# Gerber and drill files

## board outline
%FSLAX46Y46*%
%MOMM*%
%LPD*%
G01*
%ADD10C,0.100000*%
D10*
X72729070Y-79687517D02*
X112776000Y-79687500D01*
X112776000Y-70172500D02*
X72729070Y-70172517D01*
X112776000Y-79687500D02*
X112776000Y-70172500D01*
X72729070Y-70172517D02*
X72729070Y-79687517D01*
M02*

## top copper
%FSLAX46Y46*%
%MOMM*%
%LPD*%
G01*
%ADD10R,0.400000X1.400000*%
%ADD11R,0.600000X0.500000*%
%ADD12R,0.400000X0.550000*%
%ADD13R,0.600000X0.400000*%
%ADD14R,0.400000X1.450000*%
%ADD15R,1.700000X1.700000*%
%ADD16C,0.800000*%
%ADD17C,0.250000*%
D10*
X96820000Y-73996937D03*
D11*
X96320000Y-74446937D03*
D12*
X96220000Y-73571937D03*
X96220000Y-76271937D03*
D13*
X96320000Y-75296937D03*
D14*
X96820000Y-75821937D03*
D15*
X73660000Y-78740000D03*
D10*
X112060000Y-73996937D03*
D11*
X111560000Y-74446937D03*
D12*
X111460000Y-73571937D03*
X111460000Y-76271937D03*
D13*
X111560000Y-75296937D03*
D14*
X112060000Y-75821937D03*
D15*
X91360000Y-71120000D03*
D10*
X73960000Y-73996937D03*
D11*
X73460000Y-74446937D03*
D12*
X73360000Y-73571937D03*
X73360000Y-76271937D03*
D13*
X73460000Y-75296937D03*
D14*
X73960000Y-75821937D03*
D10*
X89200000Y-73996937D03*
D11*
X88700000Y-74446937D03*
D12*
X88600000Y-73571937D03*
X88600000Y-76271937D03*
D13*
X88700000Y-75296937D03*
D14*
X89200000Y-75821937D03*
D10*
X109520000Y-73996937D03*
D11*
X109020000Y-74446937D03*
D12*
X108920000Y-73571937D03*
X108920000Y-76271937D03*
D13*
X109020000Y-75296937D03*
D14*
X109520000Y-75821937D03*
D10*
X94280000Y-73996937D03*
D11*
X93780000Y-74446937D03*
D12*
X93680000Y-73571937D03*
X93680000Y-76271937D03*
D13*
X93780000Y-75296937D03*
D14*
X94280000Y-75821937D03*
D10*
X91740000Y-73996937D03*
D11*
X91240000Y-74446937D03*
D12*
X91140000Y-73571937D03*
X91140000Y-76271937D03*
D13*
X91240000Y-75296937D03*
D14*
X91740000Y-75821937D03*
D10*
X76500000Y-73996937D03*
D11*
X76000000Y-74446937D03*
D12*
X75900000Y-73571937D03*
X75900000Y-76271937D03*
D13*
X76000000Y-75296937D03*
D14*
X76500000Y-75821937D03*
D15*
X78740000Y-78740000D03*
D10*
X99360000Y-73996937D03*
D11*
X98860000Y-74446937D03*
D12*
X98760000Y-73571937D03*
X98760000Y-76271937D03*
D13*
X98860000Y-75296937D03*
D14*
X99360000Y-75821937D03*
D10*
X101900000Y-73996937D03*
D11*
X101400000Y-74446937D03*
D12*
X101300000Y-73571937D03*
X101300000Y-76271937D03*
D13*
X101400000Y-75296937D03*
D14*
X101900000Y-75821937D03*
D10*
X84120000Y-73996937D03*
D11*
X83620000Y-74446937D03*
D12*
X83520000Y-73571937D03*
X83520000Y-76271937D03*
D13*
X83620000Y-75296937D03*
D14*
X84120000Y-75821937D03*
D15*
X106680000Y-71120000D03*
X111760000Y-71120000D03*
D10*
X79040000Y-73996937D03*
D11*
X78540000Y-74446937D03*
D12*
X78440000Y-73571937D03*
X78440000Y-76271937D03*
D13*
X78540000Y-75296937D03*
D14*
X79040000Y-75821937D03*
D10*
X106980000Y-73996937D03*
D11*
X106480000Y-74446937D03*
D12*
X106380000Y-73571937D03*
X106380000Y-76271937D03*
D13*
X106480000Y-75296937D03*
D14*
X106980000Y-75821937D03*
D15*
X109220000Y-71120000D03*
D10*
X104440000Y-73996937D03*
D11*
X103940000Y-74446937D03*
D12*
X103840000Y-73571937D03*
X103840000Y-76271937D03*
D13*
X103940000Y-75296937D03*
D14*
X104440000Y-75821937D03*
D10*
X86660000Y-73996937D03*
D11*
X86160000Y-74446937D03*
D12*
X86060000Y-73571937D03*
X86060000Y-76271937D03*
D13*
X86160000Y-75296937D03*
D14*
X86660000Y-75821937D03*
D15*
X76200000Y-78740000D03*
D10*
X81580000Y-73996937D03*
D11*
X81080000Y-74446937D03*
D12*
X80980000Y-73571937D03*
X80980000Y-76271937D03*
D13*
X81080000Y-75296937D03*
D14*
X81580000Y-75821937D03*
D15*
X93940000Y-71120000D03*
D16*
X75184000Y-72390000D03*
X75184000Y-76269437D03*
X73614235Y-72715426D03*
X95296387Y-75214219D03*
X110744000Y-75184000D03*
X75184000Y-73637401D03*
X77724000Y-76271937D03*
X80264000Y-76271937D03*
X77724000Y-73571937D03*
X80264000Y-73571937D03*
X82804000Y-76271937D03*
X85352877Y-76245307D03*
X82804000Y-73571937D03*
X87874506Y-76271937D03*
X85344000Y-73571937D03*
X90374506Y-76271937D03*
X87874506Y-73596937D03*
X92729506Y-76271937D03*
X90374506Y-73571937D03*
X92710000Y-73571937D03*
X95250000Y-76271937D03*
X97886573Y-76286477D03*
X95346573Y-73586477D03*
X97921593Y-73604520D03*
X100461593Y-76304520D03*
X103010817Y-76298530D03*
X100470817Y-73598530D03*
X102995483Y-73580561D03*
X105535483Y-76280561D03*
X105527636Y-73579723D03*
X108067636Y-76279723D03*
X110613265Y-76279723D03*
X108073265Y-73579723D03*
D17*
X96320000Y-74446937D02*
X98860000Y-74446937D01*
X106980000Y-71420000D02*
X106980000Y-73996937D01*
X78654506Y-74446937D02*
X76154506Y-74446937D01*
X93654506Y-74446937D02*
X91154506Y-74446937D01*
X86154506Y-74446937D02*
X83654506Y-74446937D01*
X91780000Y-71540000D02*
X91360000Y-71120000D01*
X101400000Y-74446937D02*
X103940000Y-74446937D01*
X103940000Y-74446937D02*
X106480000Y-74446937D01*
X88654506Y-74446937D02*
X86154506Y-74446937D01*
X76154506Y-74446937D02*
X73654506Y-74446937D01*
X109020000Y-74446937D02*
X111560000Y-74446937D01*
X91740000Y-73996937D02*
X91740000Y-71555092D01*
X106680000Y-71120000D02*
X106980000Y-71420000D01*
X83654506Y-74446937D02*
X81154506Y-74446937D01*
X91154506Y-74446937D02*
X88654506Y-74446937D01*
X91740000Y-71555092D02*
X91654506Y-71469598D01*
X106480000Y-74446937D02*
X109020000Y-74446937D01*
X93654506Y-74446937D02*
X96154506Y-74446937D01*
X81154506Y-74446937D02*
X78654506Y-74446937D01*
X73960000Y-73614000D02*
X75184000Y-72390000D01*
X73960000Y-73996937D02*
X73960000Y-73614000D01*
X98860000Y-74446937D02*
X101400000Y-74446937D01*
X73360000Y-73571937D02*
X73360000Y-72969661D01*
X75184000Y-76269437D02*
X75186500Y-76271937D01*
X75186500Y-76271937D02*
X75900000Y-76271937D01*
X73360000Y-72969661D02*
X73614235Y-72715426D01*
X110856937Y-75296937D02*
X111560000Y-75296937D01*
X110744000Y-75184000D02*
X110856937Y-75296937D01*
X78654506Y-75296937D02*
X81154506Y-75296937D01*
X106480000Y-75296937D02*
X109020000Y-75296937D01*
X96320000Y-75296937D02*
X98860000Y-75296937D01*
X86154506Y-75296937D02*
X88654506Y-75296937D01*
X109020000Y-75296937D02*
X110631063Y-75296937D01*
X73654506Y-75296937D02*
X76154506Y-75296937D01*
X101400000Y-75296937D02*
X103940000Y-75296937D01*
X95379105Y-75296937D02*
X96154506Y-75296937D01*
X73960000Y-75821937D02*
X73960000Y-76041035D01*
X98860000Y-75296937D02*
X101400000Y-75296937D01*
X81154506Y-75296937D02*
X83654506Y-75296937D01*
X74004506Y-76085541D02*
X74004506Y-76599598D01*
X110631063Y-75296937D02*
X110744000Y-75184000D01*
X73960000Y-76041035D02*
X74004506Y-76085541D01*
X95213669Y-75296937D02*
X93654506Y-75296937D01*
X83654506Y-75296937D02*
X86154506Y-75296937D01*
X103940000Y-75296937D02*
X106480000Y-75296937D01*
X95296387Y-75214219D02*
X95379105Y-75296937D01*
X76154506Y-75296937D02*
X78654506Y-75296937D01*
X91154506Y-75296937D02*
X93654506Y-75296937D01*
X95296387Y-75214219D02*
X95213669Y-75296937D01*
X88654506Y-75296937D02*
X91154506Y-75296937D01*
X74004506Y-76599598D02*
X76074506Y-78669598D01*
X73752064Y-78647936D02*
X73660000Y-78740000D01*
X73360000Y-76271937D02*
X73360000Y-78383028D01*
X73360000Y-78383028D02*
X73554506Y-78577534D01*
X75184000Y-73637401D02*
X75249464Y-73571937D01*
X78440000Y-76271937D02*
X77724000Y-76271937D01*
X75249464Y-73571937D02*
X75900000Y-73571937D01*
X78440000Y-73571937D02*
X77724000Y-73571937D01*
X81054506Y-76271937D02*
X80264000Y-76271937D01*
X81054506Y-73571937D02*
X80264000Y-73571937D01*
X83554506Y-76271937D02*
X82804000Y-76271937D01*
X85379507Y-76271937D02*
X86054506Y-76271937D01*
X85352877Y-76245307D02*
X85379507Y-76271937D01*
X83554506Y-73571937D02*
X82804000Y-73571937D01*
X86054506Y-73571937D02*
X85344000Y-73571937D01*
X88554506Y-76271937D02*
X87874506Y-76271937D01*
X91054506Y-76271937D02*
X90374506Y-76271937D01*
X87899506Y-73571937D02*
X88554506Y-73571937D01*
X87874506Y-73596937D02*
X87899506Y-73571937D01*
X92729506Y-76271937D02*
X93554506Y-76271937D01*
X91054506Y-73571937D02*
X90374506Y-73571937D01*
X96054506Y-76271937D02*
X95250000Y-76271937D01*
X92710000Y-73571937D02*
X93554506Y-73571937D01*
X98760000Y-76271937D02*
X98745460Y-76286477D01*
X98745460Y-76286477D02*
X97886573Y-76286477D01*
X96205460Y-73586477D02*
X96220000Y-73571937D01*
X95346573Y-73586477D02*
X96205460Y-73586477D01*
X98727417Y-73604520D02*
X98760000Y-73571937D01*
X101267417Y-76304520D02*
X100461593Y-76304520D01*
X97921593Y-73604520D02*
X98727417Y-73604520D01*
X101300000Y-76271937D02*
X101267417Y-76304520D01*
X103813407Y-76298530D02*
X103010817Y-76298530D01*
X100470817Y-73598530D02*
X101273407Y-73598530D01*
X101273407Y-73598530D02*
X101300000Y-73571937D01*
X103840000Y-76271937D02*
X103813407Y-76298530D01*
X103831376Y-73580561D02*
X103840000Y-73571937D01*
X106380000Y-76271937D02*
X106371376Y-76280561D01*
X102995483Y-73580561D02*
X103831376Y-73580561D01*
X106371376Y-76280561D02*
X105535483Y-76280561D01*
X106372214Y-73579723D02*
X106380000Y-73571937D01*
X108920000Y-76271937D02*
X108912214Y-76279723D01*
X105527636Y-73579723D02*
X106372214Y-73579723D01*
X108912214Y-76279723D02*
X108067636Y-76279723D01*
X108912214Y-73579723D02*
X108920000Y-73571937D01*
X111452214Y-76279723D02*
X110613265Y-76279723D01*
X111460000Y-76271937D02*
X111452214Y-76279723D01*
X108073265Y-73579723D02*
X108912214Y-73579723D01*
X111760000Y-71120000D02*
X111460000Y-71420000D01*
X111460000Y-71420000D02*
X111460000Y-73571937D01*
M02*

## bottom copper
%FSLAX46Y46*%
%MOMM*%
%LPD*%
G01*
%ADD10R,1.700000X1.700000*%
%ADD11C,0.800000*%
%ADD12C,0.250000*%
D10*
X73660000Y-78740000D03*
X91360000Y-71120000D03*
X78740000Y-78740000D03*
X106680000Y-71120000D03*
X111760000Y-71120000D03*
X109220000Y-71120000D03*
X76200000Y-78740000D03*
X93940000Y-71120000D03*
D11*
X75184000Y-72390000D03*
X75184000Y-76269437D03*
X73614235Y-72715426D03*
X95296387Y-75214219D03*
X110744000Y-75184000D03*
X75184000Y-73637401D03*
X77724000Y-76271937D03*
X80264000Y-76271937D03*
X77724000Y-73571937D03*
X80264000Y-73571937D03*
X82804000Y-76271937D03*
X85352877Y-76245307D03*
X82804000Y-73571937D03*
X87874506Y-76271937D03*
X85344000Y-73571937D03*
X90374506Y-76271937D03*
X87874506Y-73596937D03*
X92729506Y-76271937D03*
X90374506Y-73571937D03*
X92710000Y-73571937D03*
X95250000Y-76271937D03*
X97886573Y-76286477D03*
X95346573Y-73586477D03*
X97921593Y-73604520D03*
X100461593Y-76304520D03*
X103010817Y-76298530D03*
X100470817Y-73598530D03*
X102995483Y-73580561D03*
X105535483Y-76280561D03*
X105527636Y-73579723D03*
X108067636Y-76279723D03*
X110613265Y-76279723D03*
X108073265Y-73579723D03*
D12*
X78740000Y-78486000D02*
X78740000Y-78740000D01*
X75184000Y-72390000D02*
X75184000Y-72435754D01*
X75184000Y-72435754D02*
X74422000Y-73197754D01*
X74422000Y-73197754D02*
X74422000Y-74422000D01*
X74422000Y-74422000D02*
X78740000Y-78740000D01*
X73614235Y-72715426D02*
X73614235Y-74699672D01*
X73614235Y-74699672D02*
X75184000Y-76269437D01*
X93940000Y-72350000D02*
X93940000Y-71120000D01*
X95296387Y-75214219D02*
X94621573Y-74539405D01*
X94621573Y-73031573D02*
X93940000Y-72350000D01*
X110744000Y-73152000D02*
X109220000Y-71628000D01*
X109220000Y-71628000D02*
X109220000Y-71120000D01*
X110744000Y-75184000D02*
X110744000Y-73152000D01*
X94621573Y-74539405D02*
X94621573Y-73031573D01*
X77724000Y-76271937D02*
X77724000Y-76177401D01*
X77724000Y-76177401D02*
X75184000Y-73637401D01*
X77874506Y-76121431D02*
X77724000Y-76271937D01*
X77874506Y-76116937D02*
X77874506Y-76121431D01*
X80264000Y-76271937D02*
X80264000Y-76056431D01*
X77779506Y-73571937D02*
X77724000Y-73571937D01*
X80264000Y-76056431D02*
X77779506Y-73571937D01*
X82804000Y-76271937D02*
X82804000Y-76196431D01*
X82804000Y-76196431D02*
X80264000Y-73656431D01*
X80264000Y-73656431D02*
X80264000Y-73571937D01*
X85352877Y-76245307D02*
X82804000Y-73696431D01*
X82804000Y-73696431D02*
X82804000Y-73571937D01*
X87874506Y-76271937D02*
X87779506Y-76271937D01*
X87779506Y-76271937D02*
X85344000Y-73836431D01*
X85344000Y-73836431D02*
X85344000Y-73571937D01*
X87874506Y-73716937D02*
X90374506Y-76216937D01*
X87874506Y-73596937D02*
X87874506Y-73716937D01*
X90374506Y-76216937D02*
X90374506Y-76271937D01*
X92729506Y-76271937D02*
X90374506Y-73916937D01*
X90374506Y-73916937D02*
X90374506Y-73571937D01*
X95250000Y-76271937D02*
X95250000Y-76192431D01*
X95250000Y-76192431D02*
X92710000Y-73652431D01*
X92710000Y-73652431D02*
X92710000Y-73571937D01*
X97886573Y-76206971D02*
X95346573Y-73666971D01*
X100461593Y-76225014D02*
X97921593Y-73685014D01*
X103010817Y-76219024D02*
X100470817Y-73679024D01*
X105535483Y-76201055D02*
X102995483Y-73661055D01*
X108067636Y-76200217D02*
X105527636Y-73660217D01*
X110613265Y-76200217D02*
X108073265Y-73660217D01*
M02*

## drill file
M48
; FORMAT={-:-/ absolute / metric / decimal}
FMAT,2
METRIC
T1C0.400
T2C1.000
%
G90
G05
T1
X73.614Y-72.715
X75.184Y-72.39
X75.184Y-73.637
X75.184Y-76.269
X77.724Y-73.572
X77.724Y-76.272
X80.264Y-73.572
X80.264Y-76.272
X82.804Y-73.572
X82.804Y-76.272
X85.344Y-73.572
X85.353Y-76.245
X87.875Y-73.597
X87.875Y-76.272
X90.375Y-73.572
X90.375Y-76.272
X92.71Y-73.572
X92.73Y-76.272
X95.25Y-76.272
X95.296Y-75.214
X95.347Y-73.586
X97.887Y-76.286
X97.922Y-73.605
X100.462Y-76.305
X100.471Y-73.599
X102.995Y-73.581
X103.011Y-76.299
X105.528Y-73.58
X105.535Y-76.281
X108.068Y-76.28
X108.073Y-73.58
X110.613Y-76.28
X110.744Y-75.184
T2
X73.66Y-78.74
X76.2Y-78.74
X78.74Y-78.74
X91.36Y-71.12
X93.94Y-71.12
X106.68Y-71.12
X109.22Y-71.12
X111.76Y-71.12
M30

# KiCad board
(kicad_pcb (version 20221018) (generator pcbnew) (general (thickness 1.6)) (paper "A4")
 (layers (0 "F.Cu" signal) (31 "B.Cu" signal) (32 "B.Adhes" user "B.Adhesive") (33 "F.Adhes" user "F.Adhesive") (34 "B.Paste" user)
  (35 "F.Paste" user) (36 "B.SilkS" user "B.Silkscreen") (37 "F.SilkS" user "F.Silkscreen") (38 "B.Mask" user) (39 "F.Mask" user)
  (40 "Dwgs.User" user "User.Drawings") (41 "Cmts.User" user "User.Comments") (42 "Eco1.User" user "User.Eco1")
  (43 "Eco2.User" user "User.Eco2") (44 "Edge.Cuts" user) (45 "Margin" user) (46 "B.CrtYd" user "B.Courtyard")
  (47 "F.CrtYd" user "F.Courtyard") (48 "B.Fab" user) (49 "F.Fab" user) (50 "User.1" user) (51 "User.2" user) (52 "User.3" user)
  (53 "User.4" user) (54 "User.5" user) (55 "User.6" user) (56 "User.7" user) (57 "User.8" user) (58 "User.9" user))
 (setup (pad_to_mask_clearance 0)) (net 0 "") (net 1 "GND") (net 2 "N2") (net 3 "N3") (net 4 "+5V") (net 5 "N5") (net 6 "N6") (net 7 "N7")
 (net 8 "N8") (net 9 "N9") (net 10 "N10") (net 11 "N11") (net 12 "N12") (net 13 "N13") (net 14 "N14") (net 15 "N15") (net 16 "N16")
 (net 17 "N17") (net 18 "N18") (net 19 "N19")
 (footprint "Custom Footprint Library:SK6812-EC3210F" (layer "F.Cu") (at 96.52 74.896937 -90)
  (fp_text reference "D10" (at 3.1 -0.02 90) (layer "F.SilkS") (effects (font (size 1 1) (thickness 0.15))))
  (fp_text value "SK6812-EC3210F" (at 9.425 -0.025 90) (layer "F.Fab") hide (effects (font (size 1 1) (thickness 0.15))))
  (pad "1" smd rect (at -0.9 -0.3 90) (size 1.4 0.4) (layers "F.Cu" "F.Paste" "F.Mask") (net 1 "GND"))
  (pad "1" smd rect (at -0.45 0.2 90) (size 0.5 0.6) (layers "F.Cu" "F.Paste" "F.Mask") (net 1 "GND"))
  (pad "2" smd rect (at -1.325 0.3 90) (size 0.55 0.4) (layers "F.Cu" "F.Paste" "F.Mask") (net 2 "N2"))
  (pad "3" smd rect (at 1.375 0.3 90) (size 0.55 0.4) (layers "F.Cu" "F.Paste" "F.Mask") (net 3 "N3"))
  (pad "4" smd rect (at 0.4 0.2 90) (size 0.4 0.6) (layers "F.Cu" "F.Paste" "F.Mask") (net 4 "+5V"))
  (pad "4" smd rect (at 0.925 -0.3 90) (size 1.45 0.4) (layers "F.Cu" "F.Paste" "F.Mask") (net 4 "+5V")))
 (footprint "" (layer "F.Cu") (at 73.66 78.74)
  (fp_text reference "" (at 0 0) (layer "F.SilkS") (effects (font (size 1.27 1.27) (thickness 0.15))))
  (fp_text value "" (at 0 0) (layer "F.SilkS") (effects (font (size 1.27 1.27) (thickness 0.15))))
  (pad "1" thru_hole rect (at 0 0) (size 1.7 1.7) (drill 1) (layers "*.Cu" "*.Mask") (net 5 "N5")))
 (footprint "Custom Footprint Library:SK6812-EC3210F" (layer "F.Cu") (at 111.76 74.896937 -90)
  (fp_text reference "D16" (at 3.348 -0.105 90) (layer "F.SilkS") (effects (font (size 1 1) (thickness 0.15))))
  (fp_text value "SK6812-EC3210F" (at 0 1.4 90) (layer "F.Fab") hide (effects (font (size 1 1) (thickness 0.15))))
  (pad "1" smd rect (at -0.9 -0.3 90) (size 1.4 0.4) (layers "F.Cu" "F.Paste" "F.Mask") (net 1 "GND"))
  (pad "1" smd rect (at -0.45 0.2 90) (size 0.5 0.6) (layers "F.Cu" "F.Paste" "F.Mask") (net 1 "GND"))
  (pad "2" smd rect (at -1.325 0.3 90) (size 0.55 0.4) (layers "F.Cu" "F.Paste" "F.Mask") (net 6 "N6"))
  (pad "3" smd rect (at 1.375 0.3 90) (size 0.55 0.4) (layers "F.Cu" "F.Paste" "F.Mask") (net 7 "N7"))
  (pad "4" smd rect (at 0.4 0.2 90) (size 0.4 0.6) (layers "F.Cu" "F.Paste" "F.Mask") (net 4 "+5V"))
  (pad "4" smd rect (at 0.925 -0.3 90) (size 1.45 0.4) (layers "F.Cu" "F.Paste" "F.Mask") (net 4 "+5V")))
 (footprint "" (layer "F.Cu") (at 91.44 71.12)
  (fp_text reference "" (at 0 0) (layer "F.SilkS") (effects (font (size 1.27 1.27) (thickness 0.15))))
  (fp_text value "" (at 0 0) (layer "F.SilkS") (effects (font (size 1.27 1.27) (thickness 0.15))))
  (pad "1" thru_hole rect (at -0.08 0) (size 1.7 1.7) (drill 1) (layers "*.Cu" "*.Mask") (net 1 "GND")))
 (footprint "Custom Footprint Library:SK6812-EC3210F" (layer "F.Cu") (at 73.66 74.896937 -90)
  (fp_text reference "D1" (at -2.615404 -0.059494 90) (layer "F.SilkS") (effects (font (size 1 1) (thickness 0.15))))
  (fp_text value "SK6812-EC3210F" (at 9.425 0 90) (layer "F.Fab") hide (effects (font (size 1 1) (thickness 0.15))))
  (pad "1" smd rect (at -0.9 -0.3 90) (size 1.4 0.4) (layers "F.Cu" "F.Paste" "F.Mask") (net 1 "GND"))
  (pad "1" smd rect (at -0.45 0.2 90) (size 0.5 0.6) (layers "F.Cu" "F.Paste" "F.Mask") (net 1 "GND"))
  (pad "2" smd rect (at -1.325 0.3 90) (size 0.55 0.4) (layers "F.Cu" "F.Paste" "F.Mask") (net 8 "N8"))
  (pad "3" smd rect (at 1.375 0.3 90) (size 0.55 0.4) (layers "F.Cu" "F.Paste" "F.Mask") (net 5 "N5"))
  (pad "4" smd rect (at 0.4 0.2 90) (size 0.4 0.6) (layers "F.Cu" "F.Paste" "F.Mask") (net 4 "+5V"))
  (pad "4" smd rect (at 0.925 -0.3 90) (size 1.45 0.4) (layers "F.Cu" "F.Paste" "F.Mask") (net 4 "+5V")))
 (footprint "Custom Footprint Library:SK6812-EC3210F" (layer "F.Cu") (at 88.9 74.896937 -90)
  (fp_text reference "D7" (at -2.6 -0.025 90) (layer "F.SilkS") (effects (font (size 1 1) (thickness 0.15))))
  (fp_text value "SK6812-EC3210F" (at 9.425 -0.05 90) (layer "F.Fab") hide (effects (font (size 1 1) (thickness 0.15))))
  (pad "1" smd rect (at -0.9 -0.3 90) (size 1.4 0.4) (layers "F.Cu" "F.Paste" "F.Mask") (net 1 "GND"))
  (pad "1" smd rect (at -0.45 0.2 90) (size 0.5 0.6) (layers "F.Cu" "F.Paste" "F.Mask") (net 1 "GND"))
  (pad "2" smd rect (at -1.325 0.3 90) (size 0.55 0.4) (layers "F.Cu" "F.Paste" "F.Mask") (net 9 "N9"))
  (pad "3" smd rect (at 1.375 0.3 90) (size 0.55 0.4) (layers "F.Cu" "F.Paste" "F.Mask") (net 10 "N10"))
  (pad "4" smd rect (at 0.4 0.2 90) (size 0.4 0.6) (layers "F.Cu" "F.Paste" "F.Mask") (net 4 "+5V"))
  (pad "4" smd rect (at 0.925 -0.3 90) (size 1.45 0.4) (layers "F.Cu" "F.Paste" "F.Mask") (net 4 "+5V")))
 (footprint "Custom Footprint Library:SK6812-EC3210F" (layer "F.Cu") (at 109.22 74.896937 -90)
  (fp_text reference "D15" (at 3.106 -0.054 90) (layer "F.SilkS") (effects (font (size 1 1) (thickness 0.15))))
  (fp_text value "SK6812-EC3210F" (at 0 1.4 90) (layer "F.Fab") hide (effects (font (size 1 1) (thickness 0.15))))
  (pad "1" smd rect (at -0.9 -0.3 90) (size 1.4 0.4) (layers "F.Cu" "F.Paste" "F.Mask") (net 1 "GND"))
  (pad "1" smd rect (at -0.45 0.2 90) (size 0.5 0.6) (layers "F.Cu" "F.Paste" "F.Mask") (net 1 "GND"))
  (pad "2" smd rect (at -1.325 0.3 90) (size 0.55 0.4) (layers "F.Cu" "F.Paste" "F.Mask") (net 7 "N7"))
  (pad "3" smd rect (at 1.375 0.3 90) (size 0.55 0.4) (layers "F.Cu" "F.Paste" "F.Mask") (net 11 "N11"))
  (pad "4" smd rect (at 0.4 0.2 90) (size 0.4 0.6) (layers "F.Cu" "F.Paste" "F.Mask") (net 4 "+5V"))
  (pad "4" smd rect (at 0.925 -0.3 90) (size 1.45 0.4) (layers "F.Cu" "F.Paste" "F.Mask") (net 4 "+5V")))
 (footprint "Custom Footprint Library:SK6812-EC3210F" (layer "F.Cu") (at 93.98 74.896937 -90)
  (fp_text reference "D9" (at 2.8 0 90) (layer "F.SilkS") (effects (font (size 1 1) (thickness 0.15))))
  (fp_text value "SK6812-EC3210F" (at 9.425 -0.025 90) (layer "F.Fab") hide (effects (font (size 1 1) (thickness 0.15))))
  (pad "1" smd rect (at -0.9 -0.3 90) (size 1.4 0.4) (layers "F.Cu" "F.Paste" "F.Mask") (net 1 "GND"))
  (pad "1" smd rect (at -0.45 0.2 90) (size 0.5 0.6) (layers "F.Cu" "F.Paste" "F.Mask") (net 1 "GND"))
  (pad "2" smd rect (at -1.325 0.3 90) (size 0.55 0.4) (layers "F.Cu" "F.Paste" "F.Mask") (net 3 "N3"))
  (pad "3" smd rect (at 1.375 0.3 90) (size 0.55 0.4) (layers "F.Cu" "F.Paste" "F.Mask") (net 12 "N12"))
  (pad "4" smd rect (at 0.4 0.2 90) (size 0.4 0.6) (layers "F.Cu" "F.Paste" "F.Mask") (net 4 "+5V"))
  (pad "4" smd rect (at 0.925 -0.3 90) (size 1.45 0.4) (layers "F.Cu" "F.Paste" "F.Mask") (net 4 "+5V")))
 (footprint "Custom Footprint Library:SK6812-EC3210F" (layer "F.Cu") (at 91.44 74.896937 -90)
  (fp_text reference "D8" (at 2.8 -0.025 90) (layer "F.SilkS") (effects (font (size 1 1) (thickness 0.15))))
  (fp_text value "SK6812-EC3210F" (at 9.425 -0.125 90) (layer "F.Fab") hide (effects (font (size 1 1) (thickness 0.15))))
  (pad "1" smd rect (at -0.9 -0.3 90) (size 1.4 0.4) (layers "F.Cu" "F.Paste" "F.Mask") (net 1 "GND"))
  (pad "1" smd rect (at -0.45 0.2 90) (size 0.5 0.6) (layers "F.Cu" "F.Paste" "F.Mask") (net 1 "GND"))
  (pad "2" smd rect (at -1.325 0.3 90) (size 0.55 0.4) (layers "F.Cu" "F.Paste" "F.Mask") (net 12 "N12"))
  (pad "3" smd rect (at 1.375 0.3 90) (size 0.55 0.4) (layers "F.Cu" "F.Paste" "F.Mask") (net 9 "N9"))
  (pad "4" smd rect (at 0.4 0.2 90) (size 0.4 0.6) (layers "F.Cu" "F.Paste" "F.Mask") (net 4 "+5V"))
  (pad "4" smd rect (at 0.925 -0.3 90) (size 1.45 0.4) (layers "F.Cu" "F.Paste" "F.Mask") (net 4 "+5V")))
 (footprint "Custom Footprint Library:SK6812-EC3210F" (layer "F.Cu") (at 76.2 74.896937 -90)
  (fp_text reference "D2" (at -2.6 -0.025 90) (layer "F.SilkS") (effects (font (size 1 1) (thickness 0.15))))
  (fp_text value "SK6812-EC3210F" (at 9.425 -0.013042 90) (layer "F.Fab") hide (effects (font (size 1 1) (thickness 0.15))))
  (pad "1" smd rect (at -0.9 -0.3 90) (size 1.4 0.4) (layers "F.Cu" "F.Paste" "F.Mask") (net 1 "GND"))
  (pad "1" smd rect (at -0.45 0.2 90) (size 0.5 0.6) (layers "F.Cu" "F.Paste" "F.Mask") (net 1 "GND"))
  (pad "2" smd rect (at -1.325 0.3 90) (size 0.55 0.4) (layers "F.Cu" "F.Paste" "F.Mask") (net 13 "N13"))
  (pad "3" smd rect (at 1.375 0.3 90) (size 0.55 0.4) (layers "F.Cu" "F.Paste" "F.Mask") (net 8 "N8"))
  (pad "4" smd rect (at 0.4 0.2 90) (size 0.4 0.6) (layers "F.Cu" "F.Paste" "F.Mask") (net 4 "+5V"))
  (pad "4" smd rect (at 0.925 -0.3 90) (size 1.45 0.4) (layers "F.Cu" "F.Paste" "F.Mask") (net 4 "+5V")))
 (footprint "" (layer "F.Cu") (at 78.74 78.74)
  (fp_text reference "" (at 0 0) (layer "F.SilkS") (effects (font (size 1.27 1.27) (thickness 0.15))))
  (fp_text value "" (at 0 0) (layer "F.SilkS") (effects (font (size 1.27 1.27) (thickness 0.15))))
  (pad "1" thru_hole rect (at 0 0) (size 1.7 1.7) (drill 1) (layers "*.Cu" "*.Mask") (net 1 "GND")))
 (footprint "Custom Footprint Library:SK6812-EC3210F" (layer "F.Cu") (at 99.06 74.896937 -90)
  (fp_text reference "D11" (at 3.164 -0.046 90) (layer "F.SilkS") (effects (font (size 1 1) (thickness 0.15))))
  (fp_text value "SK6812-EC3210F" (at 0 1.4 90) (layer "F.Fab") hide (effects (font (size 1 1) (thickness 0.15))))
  (pad "1" smd rect (at -0.9 -0.3 90) (size 1.4 0.4) (layers "F.Cu" "F.Paste" "F.Mask") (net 1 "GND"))
  (pad "1" smd rect (at -0.45 0.2 90) (size 0.5 0.6) (layers "F.Cu" "F.Paste" "F.Mask") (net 1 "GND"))
  (pad "2" smd rect (at -1.325 0.3 90) (size 0.55 0.4) (layers "F.Cu" "F.Paste" "F.Mask") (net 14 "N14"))
  (pad "3" smd rect (at 1.375 0.3 90) (size 0.55 0.4) (layers "F.Cu" "F.Paste" "F.Mask") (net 2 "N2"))
  (pad "4" smd rect (at 0.4 0.2 90) (size 0.4 0.6) (layers "F.Cu" "F.Paste" "F.Mask") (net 4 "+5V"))
  (pad "4" smd rect (at 0.925 -0.3 90) (size 1.45 0.4) (layers "F.Cu" "F.Paste" "F.Mask") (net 4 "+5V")))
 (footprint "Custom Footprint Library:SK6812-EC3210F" (layer "F.Cu") (at 101.6 74.896937 -90)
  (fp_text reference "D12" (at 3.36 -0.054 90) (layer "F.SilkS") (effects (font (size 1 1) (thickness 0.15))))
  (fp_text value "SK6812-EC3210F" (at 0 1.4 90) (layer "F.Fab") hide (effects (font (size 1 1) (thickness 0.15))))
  (pad "1" smd rect (at -0.9 -0.3 90) (size 1.4 0.4) (layers "F.Cu" "F.Paste" "F.Mask") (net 1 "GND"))
  (pad "1" smd rect (at -0.45 0.2 90) (size 0.5 0.6) (layers "F.Cu" "F.Paste" "F.Mask") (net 1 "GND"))
  (pad "2" smd rect (at -1.325 0.3 90) (size 0.55 0.4) (layers "F.Cu" "F.Paste" "F.Mask") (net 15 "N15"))
  (pad "3" smd rect (at 1.375 0.3 90) (size 0.55 0.4) (layers "F.Cu" "F.Paste" "F.Mask") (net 14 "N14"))
  (pad "4" smd rect (at 0.4 0.2 90) (size 0.4 0.6) (layers "F.Cu" "F.Paste" "F.Mask") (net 4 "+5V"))
  (pad "4" smd rect (at 0.925 -0.3 90) (size 1.45 0.4) (layers "F.Cu" "F.Paste" "F.Mask") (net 4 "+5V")))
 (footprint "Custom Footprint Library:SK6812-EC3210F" (layer "F.Cu") (at 83.82 74.896937 -90)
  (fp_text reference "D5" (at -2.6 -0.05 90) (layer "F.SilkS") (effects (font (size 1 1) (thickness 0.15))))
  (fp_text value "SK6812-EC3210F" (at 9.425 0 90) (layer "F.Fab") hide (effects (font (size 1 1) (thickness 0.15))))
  (pad "1" smd rect (at -0.9 -0.3 90) (size 1.4 0.4) (layers "F.Cu" "F.Paste" "F.Mask") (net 1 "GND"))
  (pad "1" smd rect (at -0.45 0.2 90) (size 0.5 0.6) (layers "F.Cu" "F.Paste" "F.Mask") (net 1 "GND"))
  (pad "2" smd rect (at -1.325 0.3 90) (size 0.55 0.4) (layers "F.Cu" "F.Paste" "F.Mask") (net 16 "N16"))
  (pad "3" smd rect (at 1.375 0.3 90) (size 0.55 0.4) (layers "F.Cu" "F.Paste" "F.Mask") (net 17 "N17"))
  (pad "4" smd rect (at 0.4 0.2 90) (size 0.4 0.6) (layers "F.Cu" "F.Paste" "F.Mask") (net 4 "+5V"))
  (pad "4" smd rect (at 0.925 -0.3 90) (size 1.45 0.4) (layers "F.Cu" "F.Paste" "F.Mask") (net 4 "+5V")))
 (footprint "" (layer "F.Cu") (at 106.68 71.12)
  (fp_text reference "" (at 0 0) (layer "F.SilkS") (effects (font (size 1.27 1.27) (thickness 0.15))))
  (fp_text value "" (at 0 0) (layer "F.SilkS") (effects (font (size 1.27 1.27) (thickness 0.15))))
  (pad "1" thru_hole rect (at 0 0) (size 1.7 1.7) (drill 1) (layers "*.Cu" "*.Mask") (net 1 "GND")))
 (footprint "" (layer "F.Cu") (at 111.76 71.12)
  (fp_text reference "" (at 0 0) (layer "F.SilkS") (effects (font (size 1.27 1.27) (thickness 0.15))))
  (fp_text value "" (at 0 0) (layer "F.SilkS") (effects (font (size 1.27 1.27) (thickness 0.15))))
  (pad "1" thru_hole rect (at 0 0) (size 1.7 1.7) (drill 1) (layers "*.Cu" "*.Mask") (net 6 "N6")))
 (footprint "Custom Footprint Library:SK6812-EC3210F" (layer "F.Cu") (at 78.74 74.896937 -90)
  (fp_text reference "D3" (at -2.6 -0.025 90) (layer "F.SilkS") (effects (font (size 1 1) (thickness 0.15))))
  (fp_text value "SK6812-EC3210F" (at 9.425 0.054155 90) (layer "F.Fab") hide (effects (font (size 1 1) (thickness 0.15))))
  (pad "1" smd rect (at -0.9 -0.3 90) (size 1.4 0.4) (layers "F.Cu" "F.Paste" "F.Mask") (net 1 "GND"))
  (pad "1" smd rect (at -0.45 0.2 90) (size 0.5 0.6) (layers "F.Cu" "F.Paste" "F.Mask") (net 1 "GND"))
  (pad "2" smd rect (at -1.325 0.3 90) (size 0.55 0.4) (layers "F.Cu" "F.Paste" "F.Mask") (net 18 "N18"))
  (pad "3" smd rect (at 1.375 0.3 90) (size 0.55 0.4) (layers "F.Cu" "F.Paste" "F.Mask") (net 13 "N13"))
  (pad "4" smd rect (at 0.4 0.2 90) (size 0.4 0.6) (layers "F.Cu" "F.Paste" "F.Mask") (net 4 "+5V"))
  (pad "4" smd rect (at 0.925 -0.3 90) (size 1.45 0.4) (layers "F.Cu" "F.Paste" "F.Mask") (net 4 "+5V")))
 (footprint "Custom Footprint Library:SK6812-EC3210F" (layer "F.Cu") (at 106.68 74.896937 -90)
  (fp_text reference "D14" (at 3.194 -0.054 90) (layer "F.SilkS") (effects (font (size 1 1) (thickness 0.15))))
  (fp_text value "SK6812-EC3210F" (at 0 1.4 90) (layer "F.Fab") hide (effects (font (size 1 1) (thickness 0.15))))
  (pad "1" smd rect (at -0.9 -0.3 90) (size 1.4 0.4) (layers "F.Cu" "F.Paste" "F.Mask") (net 1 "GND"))
  (pad "1" smd rect (at -0.45 0.2 90) (size 0.5 0.6) (layers "F.Cu" "F.Paste" "F.Mask") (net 1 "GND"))
  (pad "2" smd rect (at -1.325 0.3 90) (size 0.55 0.4) (layers "F.Cu" "F.Paste" "F.Mask") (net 11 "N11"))
  (pad "3" smd rect (at 1.375 0.3 90) (size 0.55 0.4) (layers "F.Cu" "F.Paste" "F.Mask") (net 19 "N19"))
  (pad "4" smd rect (at 0.4 0.2 90) (size 0.4 0.6) (layers "F.Cu" "F.Paste" "F.Mask") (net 4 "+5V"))
  (pad "4" smd rect (at 0.925 -0.3 90) (size 1.45 0.4) (layers "F.Cu" "F.Paste" "F.Mask") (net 4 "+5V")))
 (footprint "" (layer "F.Cu") (at 109.22 71.12)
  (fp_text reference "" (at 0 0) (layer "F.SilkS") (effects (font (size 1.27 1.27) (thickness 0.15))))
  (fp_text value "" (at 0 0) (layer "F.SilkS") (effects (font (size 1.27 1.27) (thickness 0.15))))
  (pad "1" thru_hole rect (at 0 0) (size 1.7 1.7) (drill 1) (layers "*.Cu" "*.Mask") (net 4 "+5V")))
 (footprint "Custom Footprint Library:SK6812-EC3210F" (layer "F.Cu") (at 104.14 74.896937 -90)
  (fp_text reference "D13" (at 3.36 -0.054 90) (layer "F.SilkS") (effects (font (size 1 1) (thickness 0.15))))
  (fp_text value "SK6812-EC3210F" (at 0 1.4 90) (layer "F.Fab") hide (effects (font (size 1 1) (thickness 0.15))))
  (pad "1" smd rect (at -0.9 -0.3 90) (size 1.4 0.4) (layers "F.Cu" "F.Paste" "F.Mask") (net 1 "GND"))
  (pad "1" smd rect (at -0.45 0.2 90) (size 0.5 0.6) (layers "F.Cu" "F.Paste" "F.Mask") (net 1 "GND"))
  (pad "2" smd rect (at -1.325 0.3 90) (size 0.55 0.4) (layers "F.Cu" "F.Paste" "F.Mask") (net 19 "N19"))
  (pad "3" smd rect (at 1.375 0.3 90) (size 0.55 0.4) (layers "F.Cu" "F.Paste" "F.Mask") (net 15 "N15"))
  (pad "4" smd rect (at 0.4 0.2 90) (size 0.4 0.6) (layers "F.Cu" "F.Paste" "F.Mask") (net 4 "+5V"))
  (pad "4" smd rect (at 0.925 -0.3 90) (size 1.45 0.4) (layers "F.Cu" "F.Paste" "F.Mask") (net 4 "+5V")))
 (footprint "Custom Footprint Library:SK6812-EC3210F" (layer "F.Cu") (at 86.36 74.896937 -90)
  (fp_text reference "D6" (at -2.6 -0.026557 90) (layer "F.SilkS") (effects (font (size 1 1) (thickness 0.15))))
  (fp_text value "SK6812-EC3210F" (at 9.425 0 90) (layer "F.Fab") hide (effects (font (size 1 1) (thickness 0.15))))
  (pad "1" smd rect (at -0.9 -0.3 90) (size 1.4 0.4) (layers "F.Cu" "F.Paste" "F.Mask") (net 1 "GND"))
  (pad "1" smd rect (at -0.45 0.2 90) (size 0.5 0.6) (layers "F.Cu" "F.Paste" "F.Mask") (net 1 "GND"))
  (pad "2" smd rect (at -1.325 0.3 90) (size 0.55 0.4) (layers "F.Cu" "F.Paste" "F.Mask") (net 10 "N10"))
  (pad "3" smd rect (at 1.375 0.3 90) (size 0.55 0.4) (layers "F.Cu" "F.Paste" "F.Mask") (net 16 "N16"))
  (pad "4" smd rect (at 0.4 0.2 90) (size 0.4 0.6) (layers "F.Cu" "F.Paste" "F.Mask") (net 4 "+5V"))
  (pad "4" smd rect (at 0.925 -0.3 90) (size 1.45 0.4) (layers "F.Cu" "F.Paste" "F.Mask") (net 4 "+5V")))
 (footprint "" (layer "F.Cu") (at 76.2 78.74)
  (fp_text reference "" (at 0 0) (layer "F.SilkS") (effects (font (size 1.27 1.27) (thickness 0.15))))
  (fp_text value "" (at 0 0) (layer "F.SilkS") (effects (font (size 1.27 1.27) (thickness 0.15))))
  (pad "1" thru_hole rect (at 0 0) (size 1.7 1.7) (drill 1) (layers "*.Cu" "*.Mask") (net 4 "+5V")))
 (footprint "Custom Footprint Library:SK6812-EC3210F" (layer "F.Cu") (at 81.28 74.896937 -90)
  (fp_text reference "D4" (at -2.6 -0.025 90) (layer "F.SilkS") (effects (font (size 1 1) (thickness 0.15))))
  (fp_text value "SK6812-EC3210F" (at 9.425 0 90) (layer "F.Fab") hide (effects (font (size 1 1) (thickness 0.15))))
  (pad "1" smd rect (at -0.9 -0.3 90) (size 1.4 0.4) (layers "F.Cu" "F.Paste" "F.Mask") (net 1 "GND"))
  (pad "1" smd rect (at -0.45 0.2 90) (size 0.5 0.6) (layers "F.Cu" "F.Paste" "F.Mask") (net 1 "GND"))
  (pad "2" smd rect (at -1.325 0.3 90) (size 0.55 0.4) (layers "F.Cu" "F.Paste" "F.Mask") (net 17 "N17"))
  (pad "3" smd rect (at 1.375 0.3 90) (size 0.55 0.4) (layers "F.Cu" "F.Paste" "F.Mask") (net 18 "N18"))
  (pad "4" smd rect (at 0.4 0.2 90) (size 0.4 0.6) (layers "F.Cu" "F.Paste" "F.Mask") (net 4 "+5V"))
  (pad "4" smd rect (at 0.925 -0.3 90) (size 1.45 0.4) (layers "F.Cu" "F.Paste" "F.Mask") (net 4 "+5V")))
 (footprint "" (layer "F.Cu") (at 93.98 71.12)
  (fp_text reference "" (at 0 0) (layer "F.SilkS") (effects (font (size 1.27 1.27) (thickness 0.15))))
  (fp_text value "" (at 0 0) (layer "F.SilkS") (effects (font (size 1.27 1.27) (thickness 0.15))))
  (pad "1" thru_hole rect (at -0.04 0) (size 1.7 1.7) (drill 1) (layers "*.Cu" "*.Mask") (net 4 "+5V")))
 (gr_line (start 72.72907 79.687517) (end 112.776 79.6875) (stroke (width 0.1) (type solid)) (layer "Edge.Cuts"))
 (gr_line (start 112.776 70.1725) (end 72.72907 70.172517) (stroke (width 0.1) (type solid)) (layer "Edge.Cuts"))
 (gr_line (start 112.776 79.6875) (end 112.776 70.1725) (stroke (width 0.1) (type solid)) (layer "Edge.Cuts"))
 (gr_line (start 72.72907 70.172517) (end 72.72907 79.687517) (stroke (width 0.1) (type solid)) (layer "Edge.Cuts"))
 (segment (start 96.32 74.446937) (end 98.86 74.446937) (width 0.25) (layer "F.Cu") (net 1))
 (segment (start 106.98 71.42) (end 106.98 73.996937) (width 0.25) (layer "F.Cu") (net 1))
 (segment (start 78.654506 74.446937) (end 76.154506 74.446937) (width 0.25) (layer "F.Cu") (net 1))
 (segment (start 93.654506 74.446937) (end 91.154506 74.446937) (width 0.25) (layer "F.Cu") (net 1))
 (segment (start 86.154506 74.446937) (end 83.654506 74.446937) (width 0.25) (layer "F.Cu") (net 1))
 (segment (start 91.78 71.54) (end 91.36 71.12) (width 0.25) (layer "F.Cu") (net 1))
 (segment (start 101.4 74.446937) (end 103.94 74.446937) (width 0.25) (layer "F.Cu") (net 1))
 (segment (start 103.94 74.446937) (end 106.48 74.446937) (width 0.25) (layer "F.Cu") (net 1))
 (segment (start 88.654506 74.446937) (end 86.154506 74.446937) (width 0.25) (layer "F.Cu") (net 1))
 (segment (start 76.154506 74.446937) (end 73.654506 74.446937) (width 0.25) (layer "F.Cu") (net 1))
 (segment (start 109.02 74.446937) (end 111.56 74.446937) (width 0.25) (layer "F.Cu") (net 1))
 (segment (start 91.74 73.996937) (end 91.74 71.555092) (width 0.25) (layer "F.Cu") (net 1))
 (segment (start 106.68 71.12) (end 106.98 71.42) (width 0.25) (layer "F.Cu") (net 1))
 (segment (start 83.654506 74.446937) (end 81.154506 74.446937) (width 0.25) (layer "F.Cu") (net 1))
 (segment (start 91.154506 74.446937) (end 88.654506 74.446937) (width 0.25) (layer "F.Cu") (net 1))
 (segment (start 91.74 71.555092) (end 91.654506 71.469598) (width 0.25) (layer "F.Cu") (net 1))
 (segment (start 106.48 74.446937) (end 109.02 74.446937) (width 0.25) (layer "F.Cu") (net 1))
 (segment (start 93.654506 74.446937) (end 96.154506 74.446937) (width 0.25) (layer "F.Cu") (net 1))
 (segment (start 81.154506 74.446937) (end 78.654506 74.446937) (width 0.25) (layer "F.Cu") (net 1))
 (segment (start 73.96 73.614) (end 75.184 72.39) (width 0.25) (layer "F.Cu") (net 1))
 (segment (start 73.96 73.996937) (end 73.96 73.614) (width 0.25) (layer "F.Cu") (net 1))
 (segment (start 98.86 74.446937) (end 101.4 74.446937) (width 0.25) (layer "F.Cu") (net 1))
 (via (at 75.184 72.39) (size 0.8) (drill 0.4) (layers "F.Cu" "B.Cu") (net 1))
 (segment (start 78.74 78.486) (end 78.74 78.74) (width 0.25) (layer "B.Cu") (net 1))
 (segment (start 75.184 72.39) (end 75.184 72.435754) (width 0.25) (layer "B.Cu") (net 1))
 (segment (start 75.184 72.435754) (end 74.422 73.197754) (width 0.25) (layer "B.Cu") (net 1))
 (segment (start 74.422 73.197754) (end 74.422 74.422) (width 0.25) (layer "B.Cu") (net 1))
 (segment (start 74.422 74.422) (end 78.74 78.74) (width 0.25) (layer "B.Cu") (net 1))
 (segment (start 73.36 73.571937) (end 73.36 72.969661) (width 0.25) (layer "F.Cu") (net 8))
 (segment (start 75.184 76.269437) (end 75.1865 76.271937) (width 0.25) (layer "F.Cu") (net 8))
 (segment (start 75.1865 76.271937) (end 75.9 76.271937) (width 0.25) (layer "F.Cu") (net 8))
 (segment (start 73.36 72.969661) (end 73.614235 72.715426) (width 0.25) (layer "F.Cu") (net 8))
 (via (at 75.184 76.269437) (size 0.8) (drill 0.4) (layers "F.Cu" "B.Cu") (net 8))
 (via (at 73.614235 72.715426) (size 0.8) (drill 0.4) (layers "F.Cu" "B.Cu") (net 8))
 (segment (start 73.614235 72.715426) (end 73.614235 74.699672) (width 0.25) (layer "B.Cu") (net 8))
 (segment (start 73.614235 74.699672) (end 75.184 76.269437) (width 0.25) (layer "B.Cu") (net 8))
 (segment (start 110.856937 75.296937) (end 111.56 75.296937) (width 0.25) (layer "F.Cu") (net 4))
 (segment (start 110.744 75.184) (end 110.856937 75.296937) (width 0.25) (layer "F.Cu") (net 4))
 (segment (start 78.654506 75.296937) (end 81.154506 75.296937) (width 0.25) (layer "F.Cu") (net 4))
 (segment (start 106.48 75.296937) (end 109.02 75.296937) (width 0.25) (layer "F.Cu") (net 4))
 (segment (start 96.32 75.296937) (end 98.86 75.296937) (width 0.25) (layer "F.Cu") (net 4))
 (segment (start 86.154506 75.296937) (end 88.654506 75.296937) (width 0.25) (layer "F.Cu") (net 4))
 (segment (start 109.02 75.296937) (end 110.631063 75.296937) (width 0.25) (layer "F.Cu") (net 4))
 (segment (start 73.654506 75.296937) (end 76.154506 75.296937) (width 0.25) (layer "F.Cu") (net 4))
 (segment (start 101.4 75.296937) (end 103.94 75.296937) (width 0.25) (layer "F.Cu") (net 4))
 (segment (start 95.379105 75.296937) (end 96.154506 75.296937) (width 0.25) (layer "F.Cu") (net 4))
 (segment (start 73.96 75.821937) (end 73.96 76.041035) (width 0.25) (layer "F.Cu") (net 4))
 (segment (start 98.86 75.296937) (end 101.4 75.296937) (width 0.25) (layer "F.Cu") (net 4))
 (segment (start 81.154506 75.296937) (end 83.654506 75.296937) (width 0.25) (layer "F.Cu") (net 4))
 (segment (start 74.004506 76.085541) (end 74.004506 76.599598) (width 0.25) (layer "F.Cu") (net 4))
 (segment (start 110.631063 75.296937) (end 110.744 75.184) (width 0.25) (layer "F.Cu") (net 4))
 (segment (start 73.96 76.041035) (end 74.004506 76.085541) (width 0.25) (layer "F.Cu") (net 4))
 (segment (start 95.213669 75.296937) (end 93.654506 75.296937) (width 0.25) (layer "F.Cu") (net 4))
 (segment (start 83.654506 75.296937) (end 86.154506 75.296937) (width 0.25) (layer "F.Cu") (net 4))
 (segment (start 103.94 75.296937) (end 106.48 75.296937) (width 0.25) (layer "F.Cu") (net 4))
 (segment (start 95.296387 75.214219) (end 95.379105 75.296937) (width 0.25) (layer "F.Cu") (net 4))
 (segment (start 76.154506 75.296937) (end 78.654506 75.296937) (width 0.25) (layer "F.Cu") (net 4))
 (segment (start 91.154506 75.296937) (end 93.654506 75.296937) (width 0.25) (layer "F.Cu") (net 4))
 (segment (start 95.296387 75.214219) (end 95.213669 75.296937) (width 0.25) (layer "F.Cu") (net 4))
 (segment (start 88.654506 75.296937) (end 91.154506 75.296937) (width 0.25) (layer "F.Cu") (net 4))
 (segment (start 74.004506 76.599598) (end 76.074506 78.669598) (width 0.25) (layer "F.Cu") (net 4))
 (via (at 95.296387 75.214219) (size 0.8) (drill 0.4) (layers "F.Cu" "B.Cu") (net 4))
 (via (at 110.744 75.184) (size 0.8) (drill 0.4) (layers "F.Cu" "B.Cu") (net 4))
 (segment (start 93.94 72.35) (end 93.94 71.12) (width 0.25) (layer "B.Cu") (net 4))
 (segment (start 95.296387 75.214219) (end 94.621573 74.539405) (width 0.25) (layer "B.Cu") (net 4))
 (segment (start 94.621573 73.031573) (end 93.94 72.35) (width 0.25) (layer "B.Cu") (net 4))
 (segment (start 110.744 73.152) (end 109.22 71.628) (width 0.25) (layer "B.Cu") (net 4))
 (segment (start 109.22 71.628) (end 109.22 71.12) (width 0.25) (layer "B.Cu") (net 4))
 (segment (start 110.744 75.184) (end 110.744 73.152) (width 0.25) (layer "B.Cu") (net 4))
 (segment (start 94.621573 74.539405) (end 94.621573 73.031573) (width 0.25) (layer "B.Cu") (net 4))
 (segment (start 73.752064 78.647936) (end 73.66 78.74) (width 0.25) (layer "F.Cu") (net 5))
 (segment (start 73.36 76.271937) (end 73.36 78.383028) (width 0.25) (layer "F.Cu") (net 5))
 (segment (start 73.36 78.383028) (end 73.554506 78.577534) (width 0.25) (layer "F.Cu") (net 5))
 (segment (start 75.184 73.637401) (end 75.249464 73.571937) (width 0.25) (layer "F.Cu") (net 13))
 (segment (start 78.44 76.271937) (end 77.724 76.271937) (width 0.25) (layer "F.Cu") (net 13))
 (segment (start 75.249464 73.571937) (end 75.9 73.571937) (width 0.25) (layer "F.Cu") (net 13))
 (via (at 75.184 73.637401) (size 0.8) (drill 0.4) (layers "F.Cu" "B.Cu") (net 13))
 (via (at 77.724 76.271937) (size 0.8) (drill 0.4) (layers "F.Cu" "B.Cu") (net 13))
 (segment (start 77.724 76.271937) (end 77.724 76.177401) (width 0.25) (layer "B.Cu") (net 13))
 (segment (start 77.724 76.177401) (end 75.184 73.637401) (width 0.25) (layer "B.Cu") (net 13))
 (segment (start 77.874506 76.121431) (end 77.724 76.271937) (width 0.25) (layer "B.Cu") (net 13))
 (segment (start 77.874506 76.116937) (end 77.874506 76.121431) (width 0.25) (layer "B.Cu") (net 13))
 (segment (start 78.44 73.571937) (end 77.724 73.571937) (width 0.25) (layer "F.Cu") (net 18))
 (segment (start 81.054506 76.271937) (end 80.264 76.271937) (width 0.25) (layer "F.Cu") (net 18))
 (via (at 80.264 76.271937) (size 0.8) (drill 0.4) (layers "F.Cu" "B.Cu") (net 18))
 (via (at 77.724 73.571937) (size 0.8) (drill 0.4) (layers "F.Cu" "B.Cu") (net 18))
 (segment (start 80.264 76.271937) (end 80.264 76.056431) (width 0.25) (layer "B.Cu") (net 18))
 (segment (start 77.779506 73.571937) (end 77.724 73.571937) (width 0.25) (layer "B.Cu") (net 18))
 (segment (start 80.264 76.056431) (end 77.779506 73.571937) (width 0.25) (layer "B.Cu") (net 18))
 (segment (start 81.054506 73.571937) (end 80.264 73.571937) (width 0.25) (layer "F.Cu") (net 17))
 (segment (start 83.554506 76.271937) (end 82.804 76.271937) (width 0.25) (layer "F.Cu") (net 17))
 (via (at 80.264 73.571937) (size 0.8) (drill 0.4) (layers "F.Cu" "B.Cu") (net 17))
 (via (at 82.804 76.271937) (size 0.8) (drill 0.4) (layers "F.Cu" "B.Cu") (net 17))
 (segment (start 82.804 76.271937) (end 82.804 76.196431) (width 0.25) (layer "B.Cu") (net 17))
 (segment (start 82.804 76.196431) (end 80.264 73.656431) (width 0.25) (layer "B.Cu") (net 17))
 (segment (start 80.264 73.656431) (end 80.264 73.571937) (width 0.25) (layer "B.Cu") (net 17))
 (segment (start 85.379507 76.271937) (end 86.054506 76.271937) (width 0.25) (layer "F.Cu") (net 16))
 (segment (start 85.352877 76.245307) (end 85.379507 76.271937) (width 0.25) (layer "F.Cu") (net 16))
 (segment (start 83.554506 73.571937) (end 82.804 73.571937) (width 0.25) (layer "F.Cu") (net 16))
 (via (at 85.352877 76.245307) (size 0.8) (drill 0.4) (layers "F.Cu" "B.Cu") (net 16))
 (via (at 82.804 73.571937) (size 0.8) (drill 0.4) (layers "F.Cu" "B.Cu") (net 16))
 (segment (start 85.352877 76.245307) (end 82.804 73.696431) (width 0.25) (layer "B.Cu") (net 16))
 (segment (start 82.804 73.696431) (end 82.804 73.571937) (width 0.25) (layer "B.Cu") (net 16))
 (segment (start 86.054506 73.571937) (end 85.344 73.571937) (width 0.25) (layer "F.Cu") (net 10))
 (segment (start 88.554506 76.271937) (end 87.874506 76.271937) (width 0.25) (layer "F.Cu") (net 10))
 (via (at 87.874506 76.271937) (size 0.8) (drill 0.4) (layers "F.Cu" "B.Cu") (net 10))
 (via (at 85.344 73.571937) (size 0.8) (drill 0.4) (layers "F.Cu" "B.Cu") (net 10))
 (segment (start 87.874506 76.271937) (end 87.779506 76.271937) (width 0.25) (layer "B.Cu") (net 10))
 (segment (start 87.779506 76.271937) (end 85.344 73.836431) (width 0.25) (layer "B.Cu") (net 10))
 (segment (start 85.344 73.836431) (end 85.344 73.571937) (width 0.25) (layer "B.Cu") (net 10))
 (segment (start 91.054506 76.271937) (end 90.374506 76.271937) (width 0.25) (layer "F.Cu") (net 9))
 (segment (start 87.899506 73.571937) (end 88.554506 73.571937) (width 0.25) (layer "F.Cu") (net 9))
 (segment (start 87.874506 73.596937) (end 87.899506 73.571937) (width 0.25) (layer "F.Cu") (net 9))
 (via (at 90.374506 76.271937) (size 0.8) (drill 0.4) (layers "F.Cu" "B.Cu") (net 9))
 (via (at 87.874506 73.596937) (size 0.8) (drill 0.4) (layers "F.Cu" "B.Cu") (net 9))
 (segment (start 87.874506 73.716937) (end 90.374506 76.216937) (width 0.25) (layer "B.Cu") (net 9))
 (segment (start 87.874506 73.596937) (end 87.874506 73.716937) (width 0.25) (layer "B.Cu") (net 9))
 (segment (start 90.374506 76.216937) (end 90.374506 76.271937) (width 0.25) (layer "B.Cu") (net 9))
 (segment (start 92.729506 76.271937) (end 93.554506 76.271937) (width 0.25) (layer "F.Cu") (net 12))
 (segment (start 91.054506 73.571937) (end 90.374506 73.571937) (width 0.25) (layer "F.Cu") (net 12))
 (via (at 92.729506 76.271937) (size 0.8) (drill 0.4) (layers "F.Cu" "B.Cu") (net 12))
 (via (at 90.374506 73.571937) (size 0.8) (drill 0.4) (layers "F.Cu" "B.Cu") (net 12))
 (segment (start 92.729506 76.271937) (end 90.374506 73.916937) (width 0.25) (layer "B.Cu") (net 12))
 (segment (start 90.374506 73.916937) (end 90.374506 73.571937) (width 0.25) (layer "B.Cu") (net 12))
 (segment (start 96.054506 76.271937) (end 95.25 76.271937) (width 0.25) (layer "F.Cu") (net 3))
 (segment (start 92.71 73.571937) (end 93.554506 73.571937) (width 0.25) (layer "F.Cu") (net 3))
 (via (at 92.71 73.571937) (size 0.8) (drill 0.4) (layers "F.Cu" "B.Cu") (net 3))
 (via (at 95.25 76.271937) (size 0.8) (drill 0.4) (layers "F.Cu" "B.Cu") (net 3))
 (segment (start 95.25 76.271937) (end 95.25 76.192431) (width 0.25) (layer "B.Cu") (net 3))
 (segment (start 95.25 76.192431) (end 92.71 73.652431) (width 0.25) (layer "B.Cu") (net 3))
 (segment (start 92.71 73.652431) (end 92.71 73.571937) (width 0.25) (layer "B.Cu") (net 3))
 (segment (start 98.76 76.271937) (end 98.74546 76.286477) (width 0.25) (layer "F.Cu") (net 2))
 (segment (start 98.74546 76.286477) (end 97.886573 76.286477) (width 0.25) (layer "F.Cu") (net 2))
 (segment (start 96.20546 73.586477) (end 96.22 73.571937) (width 0.25) (layer "F.Cu") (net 2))
 (segment (start 95.346573 73.586477) (end 96.20546 73.586477) (width 0.25) (layer "F.Cu") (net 2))
 (via (at 97.886573 76.286477) (size 0.8) (drill 0.4) (layers "F.Cu" "B.Cu") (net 2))
 (via (at 95.346573 73.586477) (size 0.8) (drill 0.4) (layers "F.Cu" "B.Cu") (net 2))
 (segment (start 97.886573 76.206971) (end 95.346573 73.666971) (width 0.25) (layer "B.Cu") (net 2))
 (segment (start 98.727417 73.60452) (end 98.76 73.571937) (width 0.25) (layer "F.Cu") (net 14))
 (segment (start 101.267417 76.30452) (end 100.461593 76.30452) (width 0.25) (layer "F.Cu") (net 14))
 (segment (start 97.921593 73.60452) (end 98.727417 73.60452) (width 0.25) (layer "F.Cu") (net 14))
 (segment (start 101.3 76.271937) (end 101.267417 76.30452) (width 0.25) (layer "F.Cu") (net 14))
 (via (at 97.921593 73.60452) (size 0.8) (drill 0.4) (layers "F.Cu" "B.Cu") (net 14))
 (via (at 100.461593 76.30452) (size 0.8) (drill 0.4) (layers "F.Cu" "B.Cu") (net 14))
 (segment (start 100.461593 76.225014) (end 97.921593 73.685014) (width 0.25) (layer "B.Cu") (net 14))
 (segment (start 103.813407 76.29853) (end 103.010817 76.29853) (width 0.25) (layer "F.Cu") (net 15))
 (segment (start 100.470817 73.59853) (end 101.273407 73.59853) (width 0.25) (layer "F.Cu") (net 15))
 (segment (start 101.273407 73.59853) (end 101.3 73.571937) (width 0.25) (layer "F.Cu") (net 15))
 (segment (start 103.84 76.271937) (end 103.813407 76.29853) (width 0.25) (layer "F.Cu") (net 15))
 (via (at 103.010817 76.29853) (size 0.8) (drill 0.4) (layers "F.Cu" "B.Cu") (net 15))
 (via (at 100.470817 73.59853) (size 0.8) (drill 0.4) (layers "F.Cu" "B.Cu") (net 15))
 (segment (start 103.010817 76.219024) (end 100.470817 73.679024) (width 0.25) (layer "B.Cu") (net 15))
 (segment (start 103.831376 73.580561) (end 103.84 73.571937) (width 0.25) (layer "F.Cu") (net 19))
 (segment (start 106.38 76.271937) (end 106.371376 76.280561) (width 0.25) (layer "F.Cu") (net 19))
 (segment (start 102.995483 73.580561) (end 103.831376 73.580561) (width 0.25) (layer "F.Cu") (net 19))
 (segment (start 106.371376 76.280561) (end 105.535483 76.280561) (width 0.25) (layer "F.Cu") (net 19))
 (via (at 102.995483 73.580561) (size 0.8) (drill 0.4) (layers "F.Cu" "B.Cu") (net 19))
 (via (at 105.535483 76.280561) (size 0.8) (drill 0.4) (layers "F.Cu" "B.Cu") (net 19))
 (segment (start 105.535483 76.201055) (end 102.995483 73.661055) (width 0.25) (layer "B.Cu") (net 19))
 (segment (start 106.372214 73.579723) (end 106.38 73.571937) (width 0.25) (layer "F.Cu") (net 11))
 (segment (start 108.92 76.271937) (end 108.912214 76.279723) (width 0.25) (layer "F.Cu") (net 11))
 (segment (start 105.527636 73.579723) (end 106.372214 73.579723) (width 0.25) (layer "F.Cu") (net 11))
 (segment (start 108.912214 76.279723) (end 108.067636 76.279723) (width 0.25) (layer "F.Cu") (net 11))
 (via (at 105.527636 73.579723) (size 0.8) (drill 0.4) (layers "F.Cu" "B.Cu") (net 11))
 (via (at 108.067636 76.279723) (size 0.8) (drill 0.4) (layers "F.Cu" "B.Cu") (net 11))
 (segment (start 108.067636 76.200217) (end 105.527636 73.660217) (width 0.25) (layer "B.Cu") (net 11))
 (segment (start 108.912214 73.579723) (end 108.92 73.571937) (width 0.25) (layer "F.Cu") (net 7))
 (segment (start 111.452214 76.279723) (end 110.613265 76.279723) (width 0.25) (layer "F.Cu") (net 7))
 (segment (start 111.46 76.271937) (end 111.452214 76.279723) (width 0.25) (layer "F.Cu") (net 7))
 (segment (start 108.073265 73.579723) (end 108.912214 73.579723) (width 0.25) (layer "F.Cu") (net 7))
 (via (at 110.613265 76.279723) (size 0.8) (drill 0.4) (layers "F.Cu" "B.Cu") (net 7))
 (via (at 108.073265 73.579723) (size 0.8) (drill 0.4) (layers "F.Cu" "B.Cu") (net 7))
 (segment (start 110.613265 76.200217) (end 108.073265 73.660217) (width 0.25) (layer "B.Cu") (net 7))
 (segment (start 111.76 71.12) (end 111.46 71.42) (width 0.25) (layer "F.Cu") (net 6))
 (segment (start 111.46 71.42) (end 111.46 73.571937) (width 0.25) (layer "F.Cu") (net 6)))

